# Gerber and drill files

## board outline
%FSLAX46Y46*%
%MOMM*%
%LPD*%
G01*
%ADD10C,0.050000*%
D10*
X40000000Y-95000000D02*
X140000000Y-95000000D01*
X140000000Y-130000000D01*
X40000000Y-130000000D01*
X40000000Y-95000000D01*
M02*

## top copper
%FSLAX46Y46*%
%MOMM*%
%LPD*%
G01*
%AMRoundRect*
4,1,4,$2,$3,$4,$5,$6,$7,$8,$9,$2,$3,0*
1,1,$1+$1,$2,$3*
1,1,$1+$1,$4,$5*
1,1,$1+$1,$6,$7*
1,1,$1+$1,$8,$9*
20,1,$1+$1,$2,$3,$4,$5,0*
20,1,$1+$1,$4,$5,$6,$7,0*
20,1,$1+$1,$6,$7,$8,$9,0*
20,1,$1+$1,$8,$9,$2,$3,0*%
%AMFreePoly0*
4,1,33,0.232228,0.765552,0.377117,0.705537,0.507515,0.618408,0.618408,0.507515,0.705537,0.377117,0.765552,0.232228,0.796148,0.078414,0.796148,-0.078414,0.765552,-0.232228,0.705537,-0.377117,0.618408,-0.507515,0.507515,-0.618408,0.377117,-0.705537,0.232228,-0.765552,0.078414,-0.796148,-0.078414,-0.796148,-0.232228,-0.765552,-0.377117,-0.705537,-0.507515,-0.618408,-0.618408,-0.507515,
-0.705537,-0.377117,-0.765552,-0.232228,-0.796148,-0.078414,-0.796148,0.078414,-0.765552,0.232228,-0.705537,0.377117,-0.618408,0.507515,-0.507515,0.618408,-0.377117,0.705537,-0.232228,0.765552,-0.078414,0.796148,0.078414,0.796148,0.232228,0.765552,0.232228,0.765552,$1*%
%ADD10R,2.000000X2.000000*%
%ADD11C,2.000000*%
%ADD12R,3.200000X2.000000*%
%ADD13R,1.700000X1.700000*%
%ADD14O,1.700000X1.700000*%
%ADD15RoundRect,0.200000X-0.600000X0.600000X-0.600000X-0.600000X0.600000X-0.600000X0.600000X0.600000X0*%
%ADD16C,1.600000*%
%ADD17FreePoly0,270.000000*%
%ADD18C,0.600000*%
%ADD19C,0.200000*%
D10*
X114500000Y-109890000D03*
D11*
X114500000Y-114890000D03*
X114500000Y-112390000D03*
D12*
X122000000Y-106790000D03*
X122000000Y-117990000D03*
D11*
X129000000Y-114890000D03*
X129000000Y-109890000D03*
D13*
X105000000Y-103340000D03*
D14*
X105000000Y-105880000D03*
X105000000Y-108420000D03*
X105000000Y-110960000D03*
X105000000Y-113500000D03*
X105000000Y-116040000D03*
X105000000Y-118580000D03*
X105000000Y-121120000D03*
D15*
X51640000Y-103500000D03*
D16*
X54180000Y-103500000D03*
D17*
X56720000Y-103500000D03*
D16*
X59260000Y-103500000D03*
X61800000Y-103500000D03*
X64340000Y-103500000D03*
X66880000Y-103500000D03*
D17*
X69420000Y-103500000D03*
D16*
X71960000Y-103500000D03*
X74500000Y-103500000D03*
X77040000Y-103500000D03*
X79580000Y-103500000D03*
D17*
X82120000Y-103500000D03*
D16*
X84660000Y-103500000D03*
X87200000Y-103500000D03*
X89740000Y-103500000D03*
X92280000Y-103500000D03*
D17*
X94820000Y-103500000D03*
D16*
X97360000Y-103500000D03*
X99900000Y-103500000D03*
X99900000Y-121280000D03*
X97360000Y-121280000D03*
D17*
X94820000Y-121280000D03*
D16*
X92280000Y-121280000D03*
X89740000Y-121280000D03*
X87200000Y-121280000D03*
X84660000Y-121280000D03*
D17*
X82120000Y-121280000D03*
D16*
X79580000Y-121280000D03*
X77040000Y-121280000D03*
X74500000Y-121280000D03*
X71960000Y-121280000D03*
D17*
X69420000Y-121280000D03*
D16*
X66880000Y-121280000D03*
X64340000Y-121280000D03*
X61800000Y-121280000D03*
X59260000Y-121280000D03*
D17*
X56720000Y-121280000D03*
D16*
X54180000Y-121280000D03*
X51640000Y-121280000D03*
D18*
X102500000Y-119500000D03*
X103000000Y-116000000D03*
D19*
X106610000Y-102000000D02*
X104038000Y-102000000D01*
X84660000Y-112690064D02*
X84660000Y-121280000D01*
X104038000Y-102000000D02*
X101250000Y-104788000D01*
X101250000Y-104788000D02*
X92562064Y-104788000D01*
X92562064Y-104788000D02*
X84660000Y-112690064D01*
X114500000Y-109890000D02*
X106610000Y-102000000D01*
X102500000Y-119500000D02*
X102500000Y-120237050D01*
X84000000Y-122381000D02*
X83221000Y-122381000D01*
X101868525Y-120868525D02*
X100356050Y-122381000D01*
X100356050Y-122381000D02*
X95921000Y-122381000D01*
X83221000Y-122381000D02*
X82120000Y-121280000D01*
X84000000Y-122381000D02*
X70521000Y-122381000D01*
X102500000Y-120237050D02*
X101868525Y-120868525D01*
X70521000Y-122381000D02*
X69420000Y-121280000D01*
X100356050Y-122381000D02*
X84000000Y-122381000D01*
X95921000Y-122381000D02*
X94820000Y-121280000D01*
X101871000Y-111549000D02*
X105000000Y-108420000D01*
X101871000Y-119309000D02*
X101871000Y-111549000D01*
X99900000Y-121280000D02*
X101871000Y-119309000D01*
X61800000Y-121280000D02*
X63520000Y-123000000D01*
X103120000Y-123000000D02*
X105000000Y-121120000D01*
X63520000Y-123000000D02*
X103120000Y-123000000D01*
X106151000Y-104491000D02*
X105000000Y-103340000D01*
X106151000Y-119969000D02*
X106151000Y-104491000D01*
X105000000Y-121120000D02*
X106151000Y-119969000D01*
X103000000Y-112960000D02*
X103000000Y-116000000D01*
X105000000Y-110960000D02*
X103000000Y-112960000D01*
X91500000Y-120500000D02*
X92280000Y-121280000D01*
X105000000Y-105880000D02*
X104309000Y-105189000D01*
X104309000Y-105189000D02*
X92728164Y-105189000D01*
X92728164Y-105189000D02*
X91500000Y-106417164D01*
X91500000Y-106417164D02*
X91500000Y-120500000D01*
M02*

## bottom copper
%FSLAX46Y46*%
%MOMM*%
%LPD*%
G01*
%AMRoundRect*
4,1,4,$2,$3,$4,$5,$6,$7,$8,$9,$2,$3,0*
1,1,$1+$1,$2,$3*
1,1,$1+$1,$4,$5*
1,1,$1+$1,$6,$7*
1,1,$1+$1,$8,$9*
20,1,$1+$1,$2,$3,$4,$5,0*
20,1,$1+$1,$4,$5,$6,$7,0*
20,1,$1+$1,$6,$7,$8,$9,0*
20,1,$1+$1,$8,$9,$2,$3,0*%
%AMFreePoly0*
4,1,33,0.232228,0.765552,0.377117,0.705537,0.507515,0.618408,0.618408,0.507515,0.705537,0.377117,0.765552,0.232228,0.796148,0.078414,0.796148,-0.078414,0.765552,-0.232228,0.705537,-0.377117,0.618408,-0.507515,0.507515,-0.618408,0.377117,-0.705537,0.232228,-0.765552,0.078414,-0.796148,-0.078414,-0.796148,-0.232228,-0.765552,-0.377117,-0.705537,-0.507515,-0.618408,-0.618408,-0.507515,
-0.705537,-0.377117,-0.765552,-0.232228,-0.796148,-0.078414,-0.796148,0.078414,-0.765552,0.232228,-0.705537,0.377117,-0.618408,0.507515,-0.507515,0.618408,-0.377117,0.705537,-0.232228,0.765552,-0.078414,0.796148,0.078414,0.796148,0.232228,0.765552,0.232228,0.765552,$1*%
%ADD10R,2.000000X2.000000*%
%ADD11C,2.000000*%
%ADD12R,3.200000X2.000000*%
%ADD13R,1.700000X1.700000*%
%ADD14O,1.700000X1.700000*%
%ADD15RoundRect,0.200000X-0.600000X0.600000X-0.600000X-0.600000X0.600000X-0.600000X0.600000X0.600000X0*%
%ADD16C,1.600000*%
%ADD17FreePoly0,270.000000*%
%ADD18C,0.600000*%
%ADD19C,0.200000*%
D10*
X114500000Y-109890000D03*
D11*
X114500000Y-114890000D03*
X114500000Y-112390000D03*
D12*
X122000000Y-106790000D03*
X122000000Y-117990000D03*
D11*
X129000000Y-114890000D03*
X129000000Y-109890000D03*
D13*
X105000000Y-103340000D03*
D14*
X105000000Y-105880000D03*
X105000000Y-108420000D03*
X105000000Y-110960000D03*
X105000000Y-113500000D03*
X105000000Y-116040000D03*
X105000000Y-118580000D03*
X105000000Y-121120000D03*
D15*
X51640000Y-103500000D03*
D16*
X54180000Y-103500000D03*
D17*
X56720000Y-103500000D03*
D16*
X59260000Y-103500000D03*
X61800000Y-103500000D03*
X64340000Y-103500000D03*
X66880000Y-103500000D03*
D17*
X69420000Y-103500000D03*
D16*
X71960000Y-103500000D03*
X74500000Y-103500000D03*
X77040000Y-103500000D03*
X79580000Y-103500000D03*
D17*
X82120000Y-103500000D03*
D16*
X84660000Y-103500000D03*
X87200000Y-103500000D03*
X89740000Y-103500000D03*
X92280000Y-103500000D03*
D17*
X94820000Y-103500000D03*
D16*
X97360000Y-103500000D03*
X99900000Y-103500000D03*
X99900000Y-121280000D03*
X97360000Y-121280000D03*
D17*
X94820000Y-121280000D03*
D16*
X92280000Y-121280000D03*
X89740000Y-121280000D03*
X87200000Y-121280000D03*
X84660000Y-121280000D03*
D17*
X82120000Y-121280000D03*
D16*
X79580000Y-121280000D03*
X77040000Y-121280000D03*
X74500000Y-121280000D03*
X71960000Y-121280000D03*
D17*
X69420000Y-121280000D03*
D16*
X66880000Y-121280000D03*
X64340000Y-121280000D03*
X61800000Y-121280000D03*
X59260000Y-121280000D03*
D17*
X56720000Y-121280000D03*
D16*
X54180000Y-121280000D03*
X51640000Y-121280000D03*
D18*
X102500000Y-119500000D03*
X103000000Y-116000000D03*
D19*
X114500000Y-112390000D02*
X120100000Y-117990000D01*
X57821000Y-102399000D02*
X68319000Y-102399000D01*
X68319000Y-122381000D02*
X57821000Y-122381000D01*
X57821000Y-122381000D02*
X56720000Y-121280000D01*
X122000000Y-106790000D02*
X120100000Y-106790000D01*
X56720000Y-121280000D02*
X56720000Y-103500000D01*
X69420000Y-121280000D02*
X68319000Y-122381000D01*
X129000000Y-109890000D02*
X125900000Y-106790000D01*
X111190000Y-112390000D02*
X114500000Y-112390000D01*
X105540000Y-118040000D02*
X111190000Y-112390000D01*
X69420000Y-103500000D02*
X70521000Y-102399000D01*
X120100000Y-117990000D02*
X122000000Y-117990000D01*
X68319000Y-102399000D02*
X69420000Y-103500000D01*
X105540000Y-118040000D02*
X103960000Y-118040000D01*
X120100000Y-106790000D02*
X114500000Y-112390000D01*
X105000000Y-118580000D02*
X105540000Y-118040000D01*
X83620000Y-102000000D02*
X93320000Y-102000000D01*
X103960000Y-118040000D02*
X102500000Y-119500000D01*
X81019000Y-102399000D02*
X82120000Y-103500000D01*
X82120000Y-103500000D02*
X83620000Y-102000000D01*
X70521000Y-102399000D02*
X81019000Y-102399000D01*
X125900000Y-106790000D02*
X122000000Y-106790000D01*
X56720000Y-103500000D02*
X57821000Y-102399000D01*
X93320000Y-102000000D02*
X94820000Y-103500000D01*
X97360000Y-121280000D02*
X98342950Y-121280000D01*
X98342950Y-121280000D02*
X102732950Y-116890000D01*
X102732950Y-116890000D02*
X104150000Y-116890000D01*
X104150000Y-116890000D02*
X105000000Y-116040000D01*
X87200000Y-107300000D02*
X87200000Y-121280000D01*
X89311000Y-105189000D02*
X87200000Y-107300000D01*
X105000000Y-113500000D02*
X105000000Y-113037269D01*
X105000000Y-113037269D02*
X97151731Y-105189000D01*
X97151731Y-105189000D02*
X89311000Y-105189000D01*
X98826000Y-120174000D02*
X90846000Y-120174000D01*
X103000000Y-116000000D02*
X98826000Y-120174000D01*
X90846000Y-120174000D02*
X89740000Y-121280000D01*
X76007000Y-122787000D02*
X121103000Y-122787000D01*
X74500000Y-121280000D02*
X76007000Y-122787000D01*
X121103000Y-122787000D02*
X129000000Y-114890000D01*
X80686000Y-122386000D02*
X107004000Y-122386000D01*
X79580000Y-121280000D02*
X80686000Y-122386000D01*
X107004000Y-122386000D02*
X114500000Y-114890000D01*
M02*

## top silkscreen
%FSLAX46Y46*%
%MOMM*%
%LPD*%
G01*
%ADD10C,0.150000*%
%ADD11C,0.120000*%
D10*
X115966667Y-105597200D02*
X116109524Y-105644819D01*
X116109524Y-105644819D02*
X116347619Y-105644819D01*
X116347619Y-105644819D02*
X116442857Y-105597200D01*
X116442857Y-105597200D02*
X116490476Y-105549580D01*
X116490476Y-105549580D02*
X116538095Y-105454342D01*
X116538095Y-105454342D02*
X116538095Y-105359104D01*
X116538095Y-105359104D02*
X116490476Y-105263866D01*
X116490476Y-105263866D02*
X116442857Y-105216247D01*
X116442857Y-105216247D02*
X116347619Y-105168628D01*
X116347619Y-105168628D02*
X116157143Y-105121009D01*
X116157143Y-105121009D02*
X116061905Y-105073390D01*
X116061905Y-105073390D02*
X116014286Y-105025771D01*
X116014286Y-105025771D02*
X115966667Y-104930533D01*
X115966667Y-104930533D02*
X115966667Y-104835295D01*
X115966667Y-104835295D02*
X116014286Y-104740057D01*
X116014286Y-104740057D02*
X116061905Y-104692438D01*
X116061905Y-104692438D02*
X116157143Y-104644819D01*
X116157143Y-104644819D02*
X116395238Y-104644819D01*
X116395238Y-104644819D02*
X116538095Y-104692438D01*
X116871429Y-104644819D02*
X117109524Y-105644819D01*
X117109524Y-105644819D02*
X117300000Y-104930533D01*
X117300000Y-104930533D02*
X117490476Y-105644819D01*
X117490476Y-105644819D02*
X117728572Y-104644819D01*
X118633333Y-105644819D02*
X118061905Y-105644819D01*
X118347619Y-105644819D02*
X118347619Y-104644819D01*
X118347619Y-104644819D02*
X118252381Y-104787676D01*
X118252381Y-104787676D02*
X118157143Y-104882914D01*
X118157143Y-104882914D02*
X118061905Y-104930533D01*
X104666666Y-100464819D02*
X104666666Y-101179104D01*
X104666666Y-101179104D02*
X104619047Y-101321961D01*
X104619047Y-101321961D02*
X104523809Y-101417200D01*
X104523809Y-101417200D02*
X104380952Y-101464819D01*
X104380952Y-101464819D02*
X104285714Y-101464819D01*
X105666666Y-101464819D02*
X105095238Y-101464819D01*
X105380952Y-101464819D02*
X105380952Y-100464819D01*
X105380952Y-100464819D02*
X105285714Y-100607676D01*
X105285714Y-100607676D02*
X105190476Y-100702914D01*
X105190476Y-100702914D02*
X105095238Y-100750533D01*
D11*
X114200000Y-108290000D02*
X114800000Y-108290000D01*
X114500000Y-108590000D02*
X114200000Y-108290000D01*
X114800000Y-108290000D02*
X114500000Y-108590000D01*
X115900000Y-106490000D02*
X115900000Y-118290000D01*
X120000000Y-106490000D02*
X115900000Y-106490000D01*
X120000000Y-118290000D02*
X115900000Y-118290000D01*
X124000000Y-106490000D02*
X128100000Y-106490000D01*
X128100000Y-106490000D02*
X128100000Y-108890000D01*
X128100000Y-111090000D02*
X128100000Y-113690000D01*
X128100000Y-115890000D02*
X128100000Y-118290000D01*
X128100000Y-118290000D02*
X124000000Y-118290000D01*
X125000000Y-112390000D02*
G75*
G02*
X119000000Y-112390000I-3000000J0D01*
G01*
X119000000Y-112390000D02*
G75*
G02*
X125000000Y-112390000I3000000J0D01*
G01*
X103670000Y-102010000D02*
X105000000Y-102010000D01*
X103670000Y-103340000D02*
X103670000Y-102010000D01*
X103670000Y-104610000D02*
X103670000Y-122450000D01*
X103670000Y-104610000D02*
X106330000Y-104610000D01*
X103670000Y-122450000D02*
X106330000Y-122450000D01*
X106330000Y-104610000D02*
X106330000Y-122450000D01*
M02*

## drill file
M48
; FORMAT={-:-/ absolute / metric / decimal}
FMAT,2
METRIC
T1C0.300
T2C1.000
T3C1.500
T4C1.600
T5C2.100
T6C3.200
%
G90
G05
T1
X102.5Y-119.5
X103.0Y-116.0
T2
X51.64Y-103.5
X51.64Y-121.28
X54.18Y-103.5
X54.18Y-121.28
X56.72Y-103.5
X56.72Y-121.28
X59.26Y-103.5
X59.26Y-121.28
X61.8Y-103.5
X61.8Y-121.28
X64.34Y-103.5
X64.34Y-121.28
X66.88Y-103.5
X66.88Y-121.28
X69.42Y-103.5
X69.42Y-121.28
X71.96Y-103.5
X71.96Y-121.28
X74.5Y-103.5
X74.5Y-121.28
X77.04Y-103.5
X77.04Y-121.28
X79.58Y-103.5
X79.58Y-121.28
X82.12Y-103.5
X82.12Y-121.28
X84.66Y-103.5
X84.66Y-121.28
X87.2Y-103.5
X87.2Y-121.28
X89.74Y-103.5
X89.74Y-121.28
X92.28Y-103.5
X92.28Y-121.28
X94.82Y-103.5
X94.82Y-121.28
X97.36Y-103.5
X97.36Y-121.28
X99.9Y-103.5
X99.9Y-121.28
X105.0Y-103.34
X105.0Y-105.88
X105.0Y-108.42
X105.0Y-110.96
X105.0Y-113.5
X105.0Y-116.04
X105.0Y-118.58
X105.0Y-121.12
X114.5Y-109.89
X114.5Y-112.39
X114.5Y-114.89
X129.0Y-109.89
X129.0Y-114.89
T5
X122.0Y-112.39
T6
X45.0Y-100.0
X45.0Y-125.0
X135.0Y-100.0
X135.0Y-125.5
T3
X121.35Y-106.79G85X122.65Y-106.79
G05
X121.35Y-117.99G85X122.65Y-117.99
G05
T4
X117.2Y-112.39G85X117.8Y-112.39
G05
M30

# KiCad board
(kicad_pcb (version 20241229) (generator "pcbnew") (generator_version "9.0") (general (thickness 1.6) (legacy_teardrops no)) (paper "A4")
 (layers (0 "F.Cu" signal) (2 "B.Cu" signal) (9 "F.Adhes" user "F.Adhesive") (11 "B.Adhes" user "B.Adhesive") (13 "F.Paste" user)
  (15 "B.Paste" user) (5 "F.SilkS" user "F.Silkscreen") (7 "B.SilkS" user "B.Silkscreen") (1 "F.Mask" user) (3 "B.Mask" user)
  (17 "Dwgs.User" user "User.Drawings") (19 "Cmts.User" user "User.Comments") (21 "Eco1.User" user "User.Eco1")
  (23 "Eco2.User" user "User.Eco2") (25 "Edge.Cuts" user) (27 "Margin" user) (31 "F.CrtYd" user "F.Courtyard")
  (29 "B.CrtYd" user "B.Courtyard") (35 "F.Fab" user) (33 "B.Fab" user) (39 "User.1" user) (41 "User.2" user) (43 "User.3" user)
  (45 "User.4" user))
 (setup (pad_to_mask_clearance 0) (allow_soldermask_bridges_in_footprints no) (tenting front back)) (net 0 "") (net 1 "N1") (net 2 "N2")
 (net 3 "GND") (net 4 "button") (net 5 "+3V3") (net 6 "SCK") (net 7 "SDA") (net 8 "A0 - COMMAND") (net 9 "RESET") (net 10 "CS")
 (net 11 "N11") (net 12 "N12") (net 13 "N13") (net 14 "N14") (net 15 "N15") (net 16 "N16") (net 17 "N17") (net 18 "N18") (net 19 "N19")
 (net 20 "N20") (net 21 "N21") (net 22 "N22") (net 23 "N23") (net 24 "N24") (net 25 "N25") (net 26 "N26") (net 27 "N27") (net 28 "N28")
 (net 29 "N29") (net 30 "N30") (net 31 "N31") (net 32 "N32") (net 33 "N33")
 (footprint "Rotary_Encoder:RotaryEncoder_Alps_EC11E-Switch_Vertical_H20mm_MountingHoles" (layer "F.Cu") (at 114.5 109.89)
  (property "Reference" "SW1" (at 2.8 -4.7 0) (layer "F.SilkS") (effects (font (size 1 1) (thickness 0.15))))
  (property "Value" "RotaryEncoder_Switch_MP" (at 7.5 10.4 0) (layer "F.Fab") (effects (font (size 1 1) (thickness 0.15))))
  (fp_line (start -0.3 -1.6) (end 0.3 -1.6) (stroke (width 0.12) (type solid)) (layer "F.SilkS"))
  (fp_line (start 0 -1.3) (end -0.3 -1.6) (stroke (width 0.12) (type solid)) (layer "F.SilkS"))
  (fp_line (start 0.3 -1.6) (end 0 -1.3) (stroke (width 0.12) (type solid)) (layer "F.SilkS"))
  (fp_line (start 1.4 -3.4) (end 1.4 8.4) (stroke (width 0.12) (type solid)) (layer "F.SilkS"))
  (fp_line (start 5.5 -3.4) (end 1.4 -3.4) (stroke (width 0.12) (type solid)) (layer "F.SilkS"))
  (fp_line (start 5.5 8.4) (end 1.4 8.4) (stroke (width 0.12) (type solid)) (layer "F.SilkS"))
  (fp_line (start 9.5 -3.4) (end 13.6 -3.4) (stroke (width 0.12) (type solid)) (layer "F.SilkS"))
  (fp_line (start 13.6 -3.4) (end 13.6 -1) (stroke (width 0.12) (type solid)) (layer "F.SilkS"))
  (fp_line (start 13.6 1.2) (end 13.6 3.8) (stroke (width 0.12) (type solid)) (layer "F.SilkS"))
  (fp_line (start 13.6 6) (end 13.6 8.4) (stroke (width 0.12) (type solid)) (layer "F.SilkS"))
  (fp_line (start 13.6 8.4) (end 9.5 8.4) (stroke (width 0.12) (type solid)) (layer "F.SilkS"))
  (fp_circle (center 7.5 2.5) (end 10.5 2.5) (stroke (width 0.12) (type solid)) (fill no) (layer "F.SilkS"))
  (pad "" np_thru_hole oval (at 3 2.5) (size 2.2 1.6) (drill oval 2.2 1.6) (layers "*.Mask"))
  (pad "" np_thru_hole circle (at 7.5 2.5) (size 2.1 2.1) (drill 2.1) (layers "*.Mask"))
  (pad "A" thru_hole rect (at 0 0) (size 2 2) (drill 1) (layers "*.Cu" "*.Mask") (remove_unused_layers no) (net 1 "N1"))
  (pad "B" thru_hole circle (at 0 5) (size 2 2) (drill 1) (layers "*.Cu" "*.Mask") (remove_unused_layers no) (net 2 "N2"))
  (pad "C" thru_hole circle (at 0 2.5) (size 2 2) (drill 1) (layers "*.Cu" "*.Mask") (remove_unused_layers no) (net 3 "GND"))
  (pad "MP" thru_hole rect (at 7.5 -3.1) (size 3.2 2) (drill oval 2.8 1.5) (layers "*.Cu" "*.Mask") (remove_unused_layers no) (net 3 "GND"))
  (pad "MP" thru_hole rect (at 7.5 8.1) (size 3.2 2) (drill oval 2.8 1.5) (layers "*.Cu" "*.Mask") (remove_unused_layers no) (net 3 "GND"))
  (pad "S1" thru_hole circle (at 14.5 5) (size 2 2) (drill 1) (layers "*.Cu" "*.Mask") (remove_unused_layers no) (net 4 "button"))
  (pad "S2" thru_hole circle (at 14.5 0) (size 2 2) (drill 1) (layers "*.Cu" "*.Mask") (remove_unused_layers no) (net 3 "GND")))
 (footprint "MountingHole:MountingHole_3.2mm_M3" (layer "F.Cu") (at 45 100)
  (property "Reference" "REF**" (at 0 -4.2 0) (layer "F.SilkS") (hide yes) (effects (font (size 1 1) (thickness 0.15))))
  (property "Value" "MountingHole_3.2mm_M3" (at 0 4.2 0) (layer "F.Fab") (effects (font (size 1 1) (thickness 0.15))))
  (pad "" np_thru_hole circle (at 0 0) (size 3.2 3.2) (drill 3.2) (layers "*.Cu" "*.Mask")))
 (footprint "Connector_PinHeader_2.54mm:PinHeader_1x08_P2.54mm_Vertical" (layer "F.Cu") (at 105 103.34)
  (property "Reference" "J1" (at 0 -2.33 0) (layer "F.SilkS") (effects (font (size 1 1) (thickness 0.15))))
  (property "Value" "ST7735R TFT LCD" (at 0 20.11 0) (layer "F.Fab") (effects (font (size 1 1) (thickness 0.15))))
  (fp_line (start -1.33 -1.33) (end 0 -1.33) (stroke (width 0.12) (type solid)) (layer "F.SilkS"))
  (fp_line (start -1.33 0) (end -1.33 -1.33) (stroke (width 0.12) (type solid)) (layer "F.SilkS"))
  (fp_line (start -1.33 1.27) (end -1.33 19.11) (stroke (width 0.12) (type solid)) (layer "F.SilkS"))
  (fp_line (start -1.33 1.27) (end 1.33 1.27) (stroke (width 0.12) (type solid)) (layer "F.SilkS"))
  (fp_line (start -1.33 19.11) (end 1.33 19.11) (stroke (width 0.12) (type solid)) (layer "F.SilkS"))
  (fp_line (start 1.33 1.27) (end 1.33 19.11) (stroke (width 0.12) (type solid)) (layer "F.SilkS"))
  (pad "1" thru_hole rect (at 0 0) (size 1.7 1.7) (drill 1) (layers "*.Cu" "*.Mask") (remove_unused_layers no) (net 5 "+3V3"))
  (pad "2" thru_hole oval (at 0 2.54) (size 1.7 1.7) (drill 1) (layers "*.Cu" "*.Mask") (remove_unused_layers no) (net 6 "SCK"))
  (pad "3" thru_hole oval (at 0 5.08) (size 1.7 1.7) (drill 1) (layers "*.Cu" "*.Mask") (remove_unused_layers no) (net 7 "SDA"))
  (pad "4" thru_hole oval (at 0 7.62) (size 1.7 1.7) (drill 1) (layers "*.Cu" "*.Mask") (remove_unused_layers no) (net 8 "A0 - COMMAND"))
  (pad "5" thru_hole oval (at 0 10.16) (size 1.7 1.7) (drill 1) (layers "*.Cu" "*.Mask") (remove_unused_layers no) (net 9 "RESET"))
  (pad "6" thru_hole oval (at 0 12.7) (size 1.7 1.7) (drill 1) (layers "*.Cu" "*.Mask") (remove_unused_layers no) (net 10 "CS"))
  (pad "7" thru_hole oval (at 0 15.24) (size 1.7 1.7) (drill 1) (layers "*.Cu" "*.Mask") (remove_unused_layers no) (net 3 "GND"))
  (pad "8" thru_hole oval (at 0 17.78) (size 1.7 1.7) (drill 1) (layers "*.Cu" "*.Mask") (remove_unused_layers no) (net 5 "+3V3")))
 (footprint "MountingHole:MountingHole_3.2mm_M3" (layer "F.Cu") (at 135 125.5)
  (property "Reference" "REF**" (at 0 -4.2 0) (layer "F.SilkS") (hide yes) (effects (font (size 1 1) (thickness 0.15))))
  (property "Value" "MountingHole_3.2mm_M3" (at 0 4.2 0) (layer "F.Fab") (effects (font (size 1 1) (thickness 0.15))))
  (pad "" np_thru_hole circle (at 0 0) (size 3.2 3.2) (drill 3.2) (layers "*.Cu" "*.Mask")))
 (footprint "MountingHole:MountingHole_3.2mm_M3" (layer "F.Cu") (at 45 125)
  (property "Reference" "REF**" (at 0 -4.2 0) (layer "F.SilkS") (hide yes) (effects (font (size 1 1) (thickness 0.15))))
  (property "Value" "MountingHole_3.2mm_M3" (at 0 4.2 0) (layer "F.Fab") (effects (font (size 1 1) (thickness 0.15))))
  (pad "" np_thru_hole circle (at 0 0) (size 3.2 3.2) (drill 3.2) (layers "*.Cu" "*.Mask")))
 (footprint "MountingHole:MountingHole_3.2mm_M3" (layer "F.Cu") (at 135 100)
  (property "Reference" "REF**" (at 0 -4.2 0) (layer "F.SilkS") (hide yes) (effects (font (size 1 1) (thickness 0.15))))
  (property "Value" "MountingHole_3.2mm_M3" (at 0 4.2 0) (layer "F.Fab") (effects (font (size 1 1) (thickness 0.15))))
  (pad "" np_thru_hole circle (at 0 0) (size 3.2 3.2) (drill 3.2) (layers "*.Cu" "*.Mask")))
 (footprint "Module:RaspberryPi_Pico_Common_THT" (layer "B.Cu") (at 51.64 103.5 -90)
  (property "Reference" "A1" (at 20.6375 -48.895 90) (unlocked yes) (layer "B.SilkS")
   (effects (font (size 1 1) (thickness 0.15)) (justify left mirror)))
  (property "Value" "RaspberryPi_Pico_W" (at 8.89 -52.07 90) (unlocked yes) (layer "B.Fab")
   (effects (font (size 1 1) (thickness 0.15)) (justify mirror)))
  (pad "1" thru_hole roundrect (at 0 0 270) (size 1.6 1.6) (drill 1) (layers "*.Cu" "*.Mask") (remove_unused_layers no)
   (roundrect_rratio 0.125) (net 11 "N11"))
  (pad "2" thru_hole circle (at 0 -2.54 270) (size 1.6 1.6) (drill 1) (layers "*.Cu" "*.Mask") (remove_unused_layers no) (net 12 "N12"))
  (pad "3" thru_hole custom (at 0 -5.08 270) (size 1.6 1.6) (drill 1) (layers "*.Cu" "*.Mask") (remove_unused_layers no) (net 3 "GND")
   (options (clearance outline) (anchor circle)) (primitives))
  (pad "4" thru_hole circle (at 0 -7.62 270) (size 1.6 1.6) (drill 1) (layers "*.Cu" "*.Mask") (remove_unused_layers no) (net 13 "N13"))
  (pad "5" thru_hole circle (at 0 -10.16 270) (size 1.6 1.6) (drill 1) (layers "*.Cu" "*.Mask") (remove_unused_layers no) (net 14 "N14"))
  (pad "6" thru_hole circle (at 0 -12.7 270) (size 1.6 1.6) (drill 1) (layers "*.Cu" "*.Mask") (remove_unused_layers no) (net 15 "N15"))
  (pad "7" thru_hole circle (at 0 -15.24 270) (size 1.6 1.6) (drill 1) (layers "*.Cu" "*.Mask") (remove_unused_layers no) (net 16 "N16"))
  (pad "8" thru_hole custom (at 0 -17.78 270) (size 1.6 1.6) (drill 1) (layers "*.Cu" "*.Mask") (remove_unused_layers no) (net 3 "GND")
   (options (clearance outline) (anchor circle)) (primitives))
  (pad "9" thru_hole circle (at 0 -20.32 270) (size 1.6 1.6) (drill 1) (layers "*.Cu" "*.Mask") (remove_unused_layers no) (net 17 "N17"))
  (pad "10" thru_hole circle (at 0 -22.86 270) (size 1.6 1.6) (drill 1) (layers "*.Cu" "*.Mask") (remove_unused_layers no) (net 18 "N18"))
  (pad "11" thru_hole circle (at 0 -25.4 270) (size 1.6 1.6) (drill 1) (layers "*.Cu" "*.Mask") (remove_unused_layers no) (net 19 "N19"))
  (pad "12" thru_hole circle (at 0 -27.94 270) (size 1.6 1.6) (drill 1) (layers "*.Cu" "*.Mask") (remove_unused_layers no) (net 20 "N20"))
  (pad "13" thru_hole custom (at 0 -30.48 270) (size 1.6 1.6) (drill 1) (layers "*.Cu" "*.Mask") (remove_unused_layers no) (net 3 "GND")
   (options (clearance outline) (anchor circle)) (primitives))
  (pad "14" thru_hole circle (at 0 -33.02 270) (size 1.6 1.6) (drill 1) (layers "*.Cu" "*.Mask") (remove_unused_layers no) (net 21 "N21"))
  (pad "15" thru_hole circle (at 0 -35.56 270) (size 1.6 1.6) (drill 1) (layers "*.Cu" "*.Mask") (remove_unused_layers no) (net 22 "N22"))
  (pad "16" thru_hole circle (at 0 -38.1 270) (size 1.6 1.6) (drill 1) (layers "*.Cu" "*.Mask") (remove_unused_layers no) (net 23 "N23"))
  (pad "17" thru_hole circle (at 0 -40.64 270) (size 1.6 1.6) (drill 1) (layers "*.Cu" "*.Mask") (remove_unused_layers no) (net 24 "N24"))
  (pad "18" thru_hole custom (at 0 -43.18 270) (size 1.6 1.6) (drill 1) (layers "*.Cu" "*.Mask") (remove_unused_layers no) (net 3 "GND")
   (options (clearance outline) (anchor circle)) (primitives))
  (pad "19" thru_hole circle (at 0 -45.72 270) (size 1.6 1.6) (drill 1) (layers "*.Cu" "*.Mask") (remove_unused_layers no) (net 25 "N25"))
  (pad "20" thru_hole circle (at 0 -48.26 270) (size 1.6 1.6) (drill 1) (layers "*.Cu" "*.Mask") (remove_unused_layers no) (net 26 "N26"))
  (pad "21" thru_hole circle (at 17.78 -48.26 270) (size 1.6 1.6) (drill 1) (layers "*.Cu" "*.Mask") (remove_unused_layers no) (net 7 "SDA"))
  (pad "22" thru_hole circle (at 17.78 -45.72 270) (size 1.6 1.6) (drill 1) (layers "*.Cu" "*.Mask") (remove_unused_layers no) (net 10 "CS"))
  (pad "23" thru_hole custom (at 17.78 -43.18 270) (size 1.6 1.6) (drill 1) (layers "*.Cu" "*.Mask") (remove_unused_layers no) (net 3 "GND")
   (options (clearance outline) (anchor circle)) (primitives))
  (pad "24" thru_hole circle (at 17.78 -40.64 270) (size 1.6 1.6) (drill 1) (layers "*.Cu" "*.Mask") (remove_unused_layers no) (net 6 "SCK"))
  (pad "25" thru_hole circle (at 17.78 -38.1 270) (size 1.6 1.6) (drill 1) (layers "*.Cu" "*.Mask") (remove_unused_layers no)
   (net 8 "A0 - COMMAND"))
  (pad "26" thru_hole circle (at 17.78 -35.56 270) (size 1.6 1.6) (drill 1) (layers "*.Cu" "*.Mask") (remove_unused_layers no)
   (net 9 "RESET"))
  (pad "27" thru_hole circle (at 17.78 -33.02 270) (size 1.6 1.6) (drill 1) (layers "*.Cu" "*.Mask") (remove_unused_layers no) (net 1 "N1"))
  (pad "28" thru_hole custom (at 17.78 -30.48 270) (size 1.6 1.6) (drill 1) (layers "*.Cu" "*.Mask") (remove_unused_layers no) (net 3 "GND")
   (options (clearance outline) (anchor circle)) (primitives))
  (pad "29" thru_hole circle (at 17.78 -27.94 270) (size 1.6 1.6) (drill 1) (layers "*.Cu" "*.Mask") (remove_unused_layers no) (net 2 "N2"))
  (pad "30" thru_hole circle (at 17.78 -25.4 270) (size 1.6 1.6) (drill 1) (layers "*.Cu" "*.Mask") (remove_unused_layers no) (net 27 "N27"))
  (pad "31" thru_hole circle (at 17.78 -22.86 270) (size 1.6 1.6) (drill 1) (layers "*.Cu" "*.Mask") (remove_unused_layers no)
   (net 4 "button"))
  (pad "32" thru_hole circle (at 17.78 -20.32 270) (size 1.6 1.6) (drill 1) (layers "*.Cu" "*.Mask") (remove_unused_layers no)
   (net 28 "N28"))
  (pad "33" thru_hole custom (at 17.78 -17.78 270) (size 1.6 1.6) (drill 1) (layers "*.Cu" "*.Mask") (remove_unused_layers no) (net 3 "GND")
   (options (clearance outline) (anchor circle)) (primitives))
  (pad "34" thru_hole circle (at 17.78 -15.24 270) (size 1.6 1.6) (drill 1) (layers "*.Cu" "*.Mask") (remove_unused_layers no)
   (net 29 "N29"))
  (pad "35" thru_hole circle (at 17.78 -12.7 270) (size 1.6 1.6) (drill 1) (layers "*.Cu" "*.Mask") (remove_unused_layers no) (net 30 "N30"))
  (pad "36" thru_hole circle (at 17.78 -10.16 270) (size 1.6 1.6) (drill 1) (layers "*.Cu" "*.Mask") (remove_unused_layers no)
   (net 5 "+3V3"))
  (pad "37" thru_hole circle (at 17.78 -7.62 270) (size 1.6 1.6) (drill 1) (layers "*.Cu" "*.Mask") (remove_unused_layers no) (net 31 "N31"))
  (pad "38" thru_hole custom (at 17.78 -5.08 270) (size 1.6 1.6) (drill 1) (layers "*.Cu" "*.Mask") (remove_unused_layers no) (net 3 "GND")
   (options (clearance outline) (anchor circle)) (primitives))
  (pad "39" thru_hole circle (at 17.78 -2.54 270) (size 1.6 1.6) (drill 1) (layers "*.Cu" "*.Mask") (remove_unused_layers no) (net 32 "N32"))
  (pad "40" thru_hole circle (at 17.78 0 270) (size 1.6 1.6) (drill 1) (layers "*.Cu" "*.Mask") (remove_unused_layers no) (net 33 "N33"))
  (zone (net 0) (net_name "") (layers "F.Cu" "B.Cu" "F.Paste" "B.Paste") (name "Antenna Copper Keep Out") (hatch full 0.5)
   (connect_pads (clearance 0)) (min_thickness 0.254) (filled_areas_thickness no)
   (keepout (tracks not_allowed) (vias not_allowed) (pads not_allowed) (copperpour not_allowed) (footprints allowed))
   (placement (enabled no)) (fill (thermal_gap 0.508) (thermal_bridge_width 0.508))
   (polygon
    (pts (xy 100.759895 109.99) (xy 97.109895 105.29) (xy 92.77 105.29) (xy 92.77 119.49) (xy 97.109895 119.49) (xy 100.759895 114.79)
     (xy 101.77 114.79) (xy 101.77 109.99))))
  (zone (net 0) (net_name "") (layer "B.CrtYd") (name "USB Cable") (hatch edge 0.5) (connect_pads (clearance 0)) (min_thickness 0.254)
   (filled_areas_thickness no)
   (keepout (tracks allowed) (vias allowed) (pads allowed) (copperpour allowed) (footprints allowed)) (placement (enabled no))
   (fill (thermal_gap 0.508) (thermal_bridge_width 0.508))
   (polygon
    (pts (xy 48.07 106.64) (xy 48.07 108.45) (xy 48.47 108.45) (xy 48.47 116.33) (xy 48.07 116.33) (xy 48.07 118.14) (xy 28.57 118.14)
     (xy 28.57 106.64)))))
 (gr_rect (start 40 95) (end 140 130) (stroke (width 0.05) (type default)) (fill no) (layer "Edge.Cuts"))
 (segment (start 106.61 102) (end 104.038 102) (width 0.2) (layer "F.Cu") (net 1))
 (segment (start 84.66 112.690064) (end 84.66 121.28) (width 0.2) (layer "F.Cu") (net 1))
 (segment (start 104.038 102) (end 101.25 104.788) (width 0.2) (layer "F.Cu") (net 1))
 (segment (start 101.25 104.788) (end 92.562064 104.788) (width 0.2) (layer "F.Cu") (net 1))
 (segment (start 92.562064 104.788) (end 84.66 112.690064) (width 0.2) (layer "F.Cu") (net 1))
 (segment (start 114.5 109.89) (end 106.61 102) (width 0.2) (layer "F.Cu") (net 1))
 (segment (start 102.5 119.5) (end 102.5 120.23705) (width 0.2) (layer "F.Cu") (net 3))
 (segment (start 84 122.381) (end 83.221 122.381) (width 0.2) (layer "F.Cu") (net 3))
 (segment (start 101.868525 120.868525) (end 100.35605 122.381) (width 0.2) (layer "F.Cu") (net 3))
 (segment (start 100.35605 122.381) (end 95.921 122.381) (width 0.2) (layer "F.Cu") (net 3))
 (segment (start 83.221 122.381) (end 82.12 121.28) (width 0.2) (layer "F.Cu") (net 3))
 (segment (start 84 122.381) (end 70.521 122.381) (width 0.2) (layer "F.Cu") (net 3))
 (segment (start 102.5 120.23705) (end 101.868525 120.868525) (width 0.2) (layer "F.Cu") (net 3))
 (segment (start 70.521 122.381) (end 69.42 121.28) (width 0.2) (layer "F.Cu") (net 3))
 (segment (start 100.35605 122.381) (end 84 122.381) (width 0.2) (layer "F.Cu") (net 3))
 (segment (start 95.921 122.381) (end 94.82 121.28) (width 0.2) (layer "F.Cu") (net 3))
 (via (at 102.5 119.5) (size 0.6) (drill 0.3) (layers "F.Cu" "B.Cu") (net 3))
 (segment (start 114.5 112.39) (end 120.1 117.99) (width 0.2) (layer "B.Cu") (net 3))
 (segment (start 57.821 102.399) (end 68.319 102.399) (width 0.2) (layer "B.Cu") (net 3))
 (segment (start 68.319 122.381) (end 57.821 122.381) (width 0.2) (layer "B.Cu") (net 3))
 (segment (start 57.821 122.381) (end 56.72 121.28) (width 0.2) (layer "B.Cu") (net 3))
 (segment (start 122 106.79) (end 120.1 106.79) (width 0.2) (layer "B.Cu") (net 3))
 (segment (start 56.72 121.28) (end 56.72 103.5) (width 0.2) (layer "B.Cu") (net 3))
 (segment (start 69.42 121.28) (end 68.319 122.381) (width 0.2) (layer "B.Cu") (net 3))
 (segment (start 129 109.89) (end 125.9 106.79) (width 0.2) (layer "B.Cu") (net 3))
 (segment (start 111.19 112.39) (end 114.5 112.39) (width 0.2) (layer "B.Cu") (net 3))
 (segment (start 105.54 118.04) (end 111.19 112.39) (width 0.2) (layer "B.Cu") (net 3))
 (segment (start 69.42 103.5) (end 70.521 102.399) (width 0.2) (layer "B.Cu") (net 3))
 (segment (start 120.1 117.99) (end 122 117.99) (width 0.2) (layer "B.Cu") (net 3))
 (segment (start 68.319 102.399) (end 69.42 103.5) (width 0.2) (layer "B.Cu") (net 3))
 (segment (start 105.54 118.04) (end 103.96 118.04) (width 0.2) (layer "B.Cu") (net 3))
 (segment (start 120.1 106.79) (end 114.5 112.39) (width 0.2) (layer "B.Cu") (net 3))
 (segment (start 105 118.58) (end 105.54 118.04) (width 0.2) (layer "B.Cu") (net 3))
 (segment (start 83.62 102) (end 93.32 102) (width 0.2) (layer "B.Cu") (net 3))
 (segment (start 103.96 118.04) (end 102.5 119.5) (width 0.2) (layer "B.Cu") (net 3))
 (segment (start 81.019 102.399) (end 82.12 103.5) (width 0.2) (layer "B.Cu") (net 3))
 (segment (start 82.12 103.5) (end 83.62 102) (width 0.2) (layer "B.Cu") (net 3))
 (segment (start 70.521 102.399) (end 81.019 102.399) (width 0.2) (layer "B.Cu") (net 3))
 (segment (start 125.9 106.79) (end 122 106.79) (width 0.2) (layer "B.Cu") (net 3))
 (segment (start 56.72 103.5) (end 57.821 102.399) (width 0.2) (layer "B.Cu") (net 3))
 (segment (start 93.32 102) (end 94.82 103.5) (width 0.2) (layer "B.Cu") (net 3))
 (segment (start 101.871 111.549) (end 105 108.42) (width 0.2) (layer "F.Cu") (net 7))
 (segment (start 101.871 119.309) (end 101.871 111.549) (width 0.2) (layer "F.Cu") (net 7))
 (segment (start 99.9 121.28) (end 101.871 119.309) (width 0.2) (layer "F.Cu") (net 7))
 (segment (start 61.8 121.28) (end 63.52 123) (width 0.2) (layer "F.Cu") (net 5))
 (segment (start 103.12 123) (end 105 121.12) (width 0.2) (layer "F.Cu") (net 5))
 (segment (start 63.52 123) (end 103.12 123) (width 0.2) (layer "F.Cu") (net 5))
 (segment (start 106.151 104.491) (end 105 103.34) (width 0.2) (layer "F.Cu") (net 5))
 (segment (start 106.151 119.969) (end 106.151 104.491) (width 0.2) (layer "F.Cu") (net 5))
 (segment (start 105 121.12) (end 106.151 119.969) (width 0.2) (layer "F.Cu") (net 5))
 (segment (start 97.36 121.28) (end 98.34295 121.28) (width 0.2) (layer "B.Cu") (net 10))
 (segment (start 98.34295 121.28) (end 102.73295 116.89) (width 0.2) (layer "B.Cu") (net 10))
 (segment (start 102.73295 116.89) (end 104.15 116.89) (width 0.2) (layer "B.Cu") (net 10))
 (segment (start 104.15 116.89) (end 105 116.04) (width 0.2) (layer "B.Cu") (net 10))
 (segment (start 87.2 107.3) (end 87.2 121.28) (width 0.2) (layer "B.Cu") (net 9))
 (segment (start 89.311 105.189) (end 87.2 107.3) (width 0.2) (layer "B.Cu") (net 9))
 (segment (start 105 113.5) (end 105 113.037269) (width 0.2) (layer "B.Cu") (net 9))
 (segment (start 105 113.037269) (end 97.151731 105.189) (width 0.2) (layer "B.Cu") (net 9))
 (segment (start 97.151731 105.189) (end 89.311 105.189) (width 0.2) (layer "B.Cu") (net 9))
 (segment (start 103 112.96) (end 103 116) (width 0.2) (layer "F.Cu") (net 8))
 (segment (start 105 110.96) (end 103 112.96) (width 0.2) (layer "F.Cu") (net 8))
 (via (at 103 116) (size 0.6) (drill 0.3) (layers "F.Cu" "B.Cu") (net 8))
 (segment (start 98.826 120.174) (end 90.846 120.174) (width 0.2) (layer "B.Cu") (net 8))
 (segment (start 103 116) (end 98.826 120.174) (width 0.2) (layer "B.Cu") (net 8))
 (segment (start 90.846 120.174) (end 89.74 121.28) (width 0.2) (layer "B.Cu") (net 8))
 (segment (start 76.007 122.787) (end 121.103 122.787) (width 0.2) (layer "B.Cu") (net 4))
 (segment (start 74.5 121.28) (end 76.007 122.787) (width 0.2) (layer "B.Cu") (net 4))
 (segment (start 121.103 122.787) (end 129 114.89) (width 0.2) (layer "B.Cu") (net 4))
 (segment (start 91.5 120.5) (end 92.28 121.28) (width 0.2) (layer "F.Cu") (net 6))
 (segment (start 105 105.88) (end 104.309 105.189) (width 0.2) (layer "F.Cu") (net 6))
 (segment (start 104.309 105.189) (end 92.728164 105.189) (width 0.2) (layer "F.Cu") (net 6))
 (segment (start 92.728164 105.189) (end 91.5 106.417164) (width 0.2) (layer "F.Cu") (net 6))
 (segment (start 91.5 106.417164) (end 91.5 120.5) (width 0.2) (layer "F.Cu") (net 6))
 (segment (start 80.686 122.386) (end 107.004 122.386) (width 0.2) (layer "B.Cu") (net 2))
 (segment (start 79.58 121.28) (end 80.686 122.386) (width 0.2) (layer "B.Cu") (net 2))
 (segment (start 107.004 122.386) (end 114.5 114.89) (width 0.2) (layer "B.Cu") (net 2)))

